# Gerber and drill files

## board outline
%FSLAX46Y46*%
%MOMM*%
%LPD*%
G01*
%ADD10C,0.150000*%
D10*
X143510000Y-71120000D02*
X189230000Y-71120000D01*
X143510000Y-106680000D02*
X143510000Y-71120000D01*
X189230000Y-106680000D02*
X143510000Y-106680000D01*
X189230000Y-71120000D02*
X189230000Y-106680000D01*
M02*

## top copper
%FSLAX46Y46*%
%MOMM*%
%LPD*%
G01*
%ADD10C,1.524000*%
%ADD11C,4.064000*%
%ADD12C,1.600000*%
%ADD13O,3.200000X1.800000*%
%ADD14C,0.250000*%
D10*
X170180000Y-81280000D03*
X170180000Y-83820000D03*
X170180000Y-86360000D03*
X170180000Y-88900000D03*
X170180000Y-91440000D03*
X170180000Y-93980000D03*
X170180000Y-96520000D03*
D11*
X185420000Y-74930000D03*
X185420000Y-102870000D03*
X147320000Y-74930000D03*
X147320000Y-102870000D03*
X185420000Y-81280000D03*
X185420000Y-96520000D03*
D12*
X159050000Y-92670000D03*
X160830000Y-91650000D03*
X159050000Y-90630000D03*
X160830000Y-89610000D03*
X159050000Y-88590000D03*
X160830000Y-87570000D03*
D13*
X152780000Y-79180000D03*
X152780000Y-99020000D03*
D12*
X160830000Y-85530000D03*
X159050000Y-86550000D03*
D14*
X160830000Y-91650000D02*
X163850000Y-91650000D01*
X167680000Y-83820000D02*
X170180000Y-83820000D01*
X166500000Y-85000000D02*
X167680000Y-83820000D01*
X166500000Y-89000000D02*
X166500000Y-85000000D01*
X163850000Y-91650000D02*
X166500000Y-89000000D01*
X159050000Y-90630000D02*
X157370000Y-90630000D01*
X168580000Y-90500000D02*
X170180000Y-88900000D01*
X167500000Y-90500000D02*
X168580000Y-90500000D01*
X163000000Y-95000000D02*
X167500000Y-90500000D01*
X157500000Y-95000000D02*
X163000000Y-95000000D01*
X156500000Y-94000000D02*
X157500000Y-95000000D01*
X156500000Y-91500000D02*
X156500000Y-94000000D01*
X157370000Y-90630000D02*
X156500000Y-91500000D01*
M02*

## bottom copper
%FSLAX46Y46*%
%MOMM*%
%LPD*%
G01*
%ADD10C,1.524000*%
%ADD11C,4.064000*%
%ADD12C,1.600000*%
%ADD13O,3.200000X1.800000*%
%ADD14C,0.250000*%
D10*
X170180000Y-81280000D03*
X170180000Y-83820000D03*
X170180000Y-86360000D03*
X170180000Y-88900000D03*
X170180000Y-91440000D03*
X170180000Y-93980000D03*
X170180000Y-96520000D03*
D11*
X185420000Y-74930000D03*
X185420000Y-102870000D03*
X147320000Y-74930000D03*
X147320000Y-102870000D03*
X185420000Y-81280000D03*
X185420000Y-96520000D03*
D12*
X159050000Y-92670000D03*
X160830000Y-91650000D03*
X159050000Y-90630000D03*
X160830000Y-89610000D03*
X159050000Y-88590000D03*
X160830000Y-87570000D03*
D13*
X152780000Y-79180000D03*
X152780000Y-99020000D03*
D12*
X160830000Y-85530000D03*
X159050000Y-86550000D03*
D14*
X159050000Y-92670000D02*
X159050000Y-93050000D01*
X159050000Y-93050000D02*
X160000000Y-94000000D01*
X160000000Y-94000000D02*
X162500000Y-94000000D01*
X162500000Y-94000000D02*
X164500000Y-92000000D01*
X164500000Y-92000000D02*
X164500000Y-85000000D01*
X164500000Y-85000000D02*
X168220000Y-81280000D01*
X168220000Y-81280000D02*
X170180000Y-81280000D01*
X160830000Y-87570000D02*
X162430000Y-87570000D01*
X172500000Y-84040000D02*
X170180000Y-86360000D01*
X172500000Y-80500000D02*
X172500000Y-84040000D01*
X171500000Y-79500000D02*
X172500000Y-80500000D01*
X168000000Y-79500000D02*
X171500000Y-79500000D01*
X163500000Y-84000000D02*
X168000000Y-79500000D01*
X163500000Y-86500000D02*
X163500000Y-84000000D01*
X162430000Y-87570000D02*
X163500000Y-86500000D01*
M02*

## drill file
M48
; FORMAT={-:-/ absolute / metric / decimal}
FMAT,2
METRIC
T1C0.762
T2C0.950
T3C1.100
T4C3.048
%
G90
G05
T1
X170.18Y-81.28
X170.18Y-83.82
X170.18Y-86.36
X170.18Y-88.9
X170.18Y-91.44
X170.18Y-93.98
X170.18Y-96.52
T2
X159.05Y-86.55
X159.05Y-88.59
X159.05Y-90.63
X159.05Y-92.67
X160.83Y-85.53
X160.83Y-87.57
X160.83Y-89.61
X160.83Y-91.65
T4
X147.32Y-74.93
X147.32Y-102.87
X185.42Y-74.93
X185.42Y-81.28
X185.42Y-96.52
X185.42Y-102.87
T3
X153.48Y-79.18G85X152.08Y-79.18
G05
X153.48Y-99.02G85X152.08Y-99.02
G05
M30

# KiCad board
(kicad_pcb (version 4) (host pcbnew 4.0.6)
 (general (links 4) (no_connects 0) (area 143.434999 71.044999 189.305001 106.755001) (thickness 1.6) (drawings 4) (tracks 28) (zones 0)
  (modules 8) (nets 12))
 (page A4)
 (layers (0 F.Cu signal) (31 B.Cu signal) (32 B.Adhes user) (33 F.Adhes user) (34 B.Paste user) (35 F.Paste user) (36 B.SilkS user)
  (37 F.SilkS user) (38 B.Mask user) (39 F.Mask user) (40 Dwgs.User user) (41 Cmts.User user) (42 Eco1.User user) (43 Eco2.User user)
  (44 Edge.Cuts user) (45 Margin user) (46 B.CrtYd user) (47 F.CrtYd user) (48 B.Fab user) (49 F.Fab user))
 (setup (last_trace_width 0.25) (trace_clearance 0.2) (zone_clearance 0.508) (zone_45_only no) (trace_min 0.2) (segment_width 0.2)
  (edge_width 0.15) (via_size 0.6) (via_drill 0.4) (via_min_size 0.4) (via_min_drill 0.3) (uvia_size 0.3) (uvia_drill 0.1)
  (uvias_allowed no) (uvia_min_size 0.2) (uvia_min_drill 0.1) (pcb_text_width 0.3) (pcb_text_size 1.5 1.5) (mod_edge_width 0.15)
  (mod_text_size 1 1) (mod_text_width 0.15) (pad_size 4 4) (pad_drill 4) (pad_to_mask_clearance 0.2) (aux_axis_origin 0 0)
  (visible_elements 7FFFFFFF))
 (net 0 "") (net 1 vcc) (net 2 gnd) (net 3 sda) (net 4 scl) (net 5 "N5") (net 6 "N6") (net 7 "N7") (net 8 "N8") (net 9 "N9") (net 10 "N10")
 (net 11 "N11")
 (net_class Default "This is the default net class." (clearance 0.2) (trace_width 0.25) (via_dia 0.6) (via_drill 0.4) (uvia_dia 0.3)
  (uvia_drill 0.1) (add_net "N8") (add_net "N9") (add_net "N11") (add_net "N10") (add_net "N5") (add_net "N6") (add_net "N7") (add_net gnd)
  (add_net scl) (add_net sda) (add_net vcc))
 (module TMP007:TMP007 (layer F.Cu) (at 170.18 88.9)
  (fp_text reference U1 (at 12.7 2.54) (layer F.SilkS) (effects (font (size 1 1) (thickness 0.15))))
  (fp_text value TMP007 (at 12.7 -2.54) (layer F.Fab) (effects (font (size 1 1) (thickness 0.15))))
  (pad 1 thru_hole circle (at 0 -7.62) (size 1.524 1.524) (drill 0.762) (layers *.Cu *.Mask) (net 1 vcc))
  (pad 2 thru_hole circle (at 0 -5.08) (size 1.524 1.524) (drill 0.762) (layers *.Cu *.Mask) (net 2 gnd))
  (pad 3 thru_hole circle (at 0 -2.54) (size 1.524 1.524) (drill 0.762) (layers *.Cu *.Mask) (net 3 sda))
  (pad 4 thru_hole circle (at 0 0) (size 1.524 1.524) (drill 0.762) (layers *.Cu *.Mask) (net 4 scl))
  (pad 5 thru_hole circle (at 0 2.54) (size 1.524 1.524) (drill 0.762) (layers *.Cu *.Mask) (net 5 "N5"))
  (pad 6 thru_hole circle (at 0 5.08) (size 1.524 1.524) (drill 0.762) (layers *.Cu *.Mask) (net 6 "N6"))
  (pad 7 thru_hole circle (at 0 7.62) (size 1.524 1.524) (drill 0.762) (layers *.Cu *.Mask) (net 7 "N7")))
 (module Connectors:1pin (layer F.Cu) (at 185.42 74.93)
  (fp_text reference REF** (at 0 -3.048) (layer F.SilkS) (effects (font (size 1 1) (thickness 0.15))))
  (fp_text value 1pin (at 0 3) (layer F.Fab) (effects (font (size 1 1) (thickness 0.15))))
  (pad 1 thru_hole circle (at 0 0) (size 4.064 4.064) (drill 3.048) (layers *.Cu *.Mask)))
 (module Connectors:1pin (layer F.Cu) (at 185.42 102.87)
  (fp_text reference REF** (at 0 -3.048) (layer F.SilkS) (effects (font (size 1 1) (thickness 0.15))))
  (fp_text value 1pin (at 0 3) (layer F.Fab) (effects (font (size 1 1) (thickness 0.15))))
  (pad 1 thru_hole circle (at 0 0) (size 4.064 4.064) (drill 3.048) (layers *.Cu *.Mask)))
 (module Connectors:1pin (layer F.Cu) (at 147.32 74.93)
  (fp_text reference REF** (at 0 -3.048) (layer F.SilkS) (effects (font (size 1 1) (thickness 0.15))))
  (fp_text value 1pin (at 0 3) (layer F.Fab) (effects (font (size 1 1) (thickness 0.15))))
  (pad 1 thru_hole circle (at 0 0) (size 4.064 4.064) (drill 3.048) (layers *.Cu *.Mask)))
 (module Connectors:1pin (layer F.Cu) (at 147.32 102.87)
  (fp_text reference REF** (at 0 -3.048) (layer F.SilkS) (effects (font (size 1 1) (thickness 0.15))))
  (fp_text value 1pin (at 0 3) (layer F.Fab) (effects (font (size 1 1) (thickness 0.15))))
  (pad 1 thru_hole circle (at 0 0) (size 4.064 4.064) (drill 3.048) (layers *.Cu *.Mask)))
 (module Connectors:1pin (layer F.Cu) (at 185.42 81.28)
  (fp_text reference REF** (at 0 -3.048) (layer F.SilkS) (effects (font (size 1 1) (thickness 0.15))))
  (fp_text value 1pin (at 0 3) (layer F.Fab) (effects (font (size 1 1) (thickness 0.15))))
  (pad 1 thru_hole circle (at 0 0) (size 4.064 4.064) (drill 3.048) (layers *.Cu *.Mask)))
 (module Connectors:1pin (layer F.Cu) (at 185.42 96.52)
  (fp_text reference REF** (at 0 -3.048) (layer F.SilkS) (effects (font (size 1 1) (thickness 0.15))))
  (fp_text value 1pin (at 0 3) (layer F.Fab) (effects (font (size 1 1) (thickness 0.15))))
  (pad 1 thru_hole circle (at 0 0) (size 4.064 4.064) (drill 3.048) (layers *.Cu *.Mask)))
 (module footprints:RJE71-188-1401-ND (layer F.Cu) (at 164.5 81 270)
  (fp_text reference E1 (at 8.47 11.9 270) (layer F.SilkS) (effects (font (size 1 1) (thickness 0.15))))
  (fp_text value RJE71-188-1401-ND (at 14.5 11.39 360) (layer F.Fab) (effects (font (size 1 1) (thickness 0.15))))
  (pad 1 thru_hole circle (at 11.67 5.45 270) (size 1.6 1.6) (drill 0.95) (layers *.Cu *.Mask) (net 1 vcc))
  (pad 2 thru_hole circle (at 10.65 3.67 270) (size 1.6 1.6) (drill 0.95) (layers *.Cu *.Mask) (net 2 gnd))
  (pad 3 thru_hole circle (at 9.63 5.45 270) (size 1.6 1.6) (drill 0.95) (layers *.Cu *.Mask) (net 4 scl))
  (pad 4 thru_hole circle (at 8.61 3.67 270) (size 1.6 1.6) (drill 0.95) (layers *.Cu *.Mask) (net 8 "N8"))
  (pad 5 thru_hole circle (at 7.59 5.45 270) (size 1.6 1.6) (drill 0.95) (layers *.Cu *.Mask) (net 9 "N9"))
  (pad 6 thru_hole circle (at 6.57 3.67 270) (size 1.6 1.6) (drill 0.95) (layers *.Cu *.Mask) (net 3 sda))
  (pad "" thru_hole oval (at -1.82 11.72 270) (size 1.8 3.2) (drill oval 1.1 2.5) (layers *.Cu *.Mask))
  (pad "" thru_hole oval (at 18.02 11.72 270) (size 1.8 3.2) (drill oval 1.1 2.5) (layers *.Cu *.Mask))
  (pad 8 thru_hole circle (at 4.53 3.67 270) (size 1.6 1.6) (drill 0.95) (layers *.Cu *.Mask) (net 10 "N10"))
  (pad 7 thru_hole circle (at 5.55 5.45 270) (size 1.6 1.6) (drill 0.95) (layers *.Cu *.Mask) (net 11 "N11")))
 (gr_line (start 143.51 71.12) (end 189.23 71.12) (angle 90) (layer Edge.Cuts) (width 0.15))
 (gr_line (start 143.51 106.68) (end 143.51 71.12) (angle 90) (layer Edge.Cuts) (width 0.15))
 (gr_line (start 189.23 106.68) (end 143.51 106.68) (angle 90) (layer Edge.Cuts) (width 0.15))
 (gr_line (start 189.23 71.12) (end 189.23 106.68) (angle 90) (layer Edge.Cuts) (width 0.15))
 (segment (start 159.05 92.67) (end 159.05 93.05) (width 0.25) (layer B.Cu) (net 1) (status C00000))
 (segment (start 159.05 93.05) (end 160 94) (width 0.25) (layer B.Cu) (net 1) (status 400000))
 (segment (start 160 94) (end 162.5 94) (width 0.25) (layer B.Cu) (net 1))
 (segment (start 162.5 94) (end 164.5 92) (width 0.25) (layer B.Cu) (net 1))
 (segment (start 164.5 92) (end 164.5 85) (width 0.25) (layer B.Cu) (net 1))
 (segment (start 164.5 85) (end 168.22 81.28) (width 0.25) (layer B.Cu) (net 1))
 (segment (start 168.22 81.28) (end 170.18 81.28) (width 0.25) (layer B.Cu) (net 1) (status 800000))
 (segment (start 160.83 91.65) (end 163.85 91.65) (width 0.25) (layer F.Cu) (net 2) (status 400000))
 (segment (start 167.68 83.82) (end 170.18 83.82) (width 0.25) (layer F.Cu) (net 2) (status 800000))
 (segment (start 166.5 85) (end 167.68 83.82) (width 0.25) (layer F.Cu) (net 2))
 (segment (start 166.5 89) (end 166.5 85) (width 0.25) (layer F.Cu) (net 2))
 (segment (start 163.85 91.65) (end 166.5 89) (width 0.25) (layer F.Cu) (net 2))
 (segment (start 159.05 90.63) (end 157.37 90.63) (width 0.25) (layer F.Cu) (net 4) (status 400000))
 (segment (start 168.58 90.5) (end 170.18 88.9) (width 0.25) (layer F.Cu) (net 4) (status 800000))
 (segment (start 167.5 90.5) (end 168.58 90.5) (width 0.25) (layer F.Cu) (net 4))
 (segment (start 163 95) (end 167.5 90.5) (width 0.25) (layer F.Cu) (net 4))
 (segment (start 157.5 95) (end 163 95) (width 0.25) (layer F.Cu) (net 4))
 (segment (start 156.5 94) (end 157.5 95) (width 0.25) (layer F.Cu) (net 4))
 (segment (start 156.5 91.5) (end 156.5 94) (width 0.25) (layer F.Cu) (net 4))
 (segment (start 157.37 90.63) (end 156.5 91.5) (width 0.25) (layer F.Cu) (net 4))
 (segment (start 160.83 87.57) (end 162.43 87.57) (width 0.25) (layer B.Cu) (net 3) (status 400000))
 (segment (start 172.5 84.04) (end 170.18 86.36) (width 0.25) (layer B.Cu) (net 3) (status 800000))
 (segment (start 172.5 80.5) (end 172.5 84.04) (width 0.25) (layer B.Cu) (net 3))
 (segment (start 171.5 79.5) (end 172.5 80.5) (width 0.25) (layer B.Cu) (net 3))
 (segment (start 168 79.5) (end 171.5 79.5) (width 0.25) (layer B.Cu) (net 3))
 (segment (start 163.5 84) (end 168 79.5) (width 0.25) (layer B.Cu) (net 3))
 (segment (start 163.5 86.5) (end 163.5 84) (width 0.25) (layer B.Cu) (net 3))
 (segment (start 162.43 87.57) (end 163.5 86.5) (width 0.25) (layer B.Cu) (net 3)))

